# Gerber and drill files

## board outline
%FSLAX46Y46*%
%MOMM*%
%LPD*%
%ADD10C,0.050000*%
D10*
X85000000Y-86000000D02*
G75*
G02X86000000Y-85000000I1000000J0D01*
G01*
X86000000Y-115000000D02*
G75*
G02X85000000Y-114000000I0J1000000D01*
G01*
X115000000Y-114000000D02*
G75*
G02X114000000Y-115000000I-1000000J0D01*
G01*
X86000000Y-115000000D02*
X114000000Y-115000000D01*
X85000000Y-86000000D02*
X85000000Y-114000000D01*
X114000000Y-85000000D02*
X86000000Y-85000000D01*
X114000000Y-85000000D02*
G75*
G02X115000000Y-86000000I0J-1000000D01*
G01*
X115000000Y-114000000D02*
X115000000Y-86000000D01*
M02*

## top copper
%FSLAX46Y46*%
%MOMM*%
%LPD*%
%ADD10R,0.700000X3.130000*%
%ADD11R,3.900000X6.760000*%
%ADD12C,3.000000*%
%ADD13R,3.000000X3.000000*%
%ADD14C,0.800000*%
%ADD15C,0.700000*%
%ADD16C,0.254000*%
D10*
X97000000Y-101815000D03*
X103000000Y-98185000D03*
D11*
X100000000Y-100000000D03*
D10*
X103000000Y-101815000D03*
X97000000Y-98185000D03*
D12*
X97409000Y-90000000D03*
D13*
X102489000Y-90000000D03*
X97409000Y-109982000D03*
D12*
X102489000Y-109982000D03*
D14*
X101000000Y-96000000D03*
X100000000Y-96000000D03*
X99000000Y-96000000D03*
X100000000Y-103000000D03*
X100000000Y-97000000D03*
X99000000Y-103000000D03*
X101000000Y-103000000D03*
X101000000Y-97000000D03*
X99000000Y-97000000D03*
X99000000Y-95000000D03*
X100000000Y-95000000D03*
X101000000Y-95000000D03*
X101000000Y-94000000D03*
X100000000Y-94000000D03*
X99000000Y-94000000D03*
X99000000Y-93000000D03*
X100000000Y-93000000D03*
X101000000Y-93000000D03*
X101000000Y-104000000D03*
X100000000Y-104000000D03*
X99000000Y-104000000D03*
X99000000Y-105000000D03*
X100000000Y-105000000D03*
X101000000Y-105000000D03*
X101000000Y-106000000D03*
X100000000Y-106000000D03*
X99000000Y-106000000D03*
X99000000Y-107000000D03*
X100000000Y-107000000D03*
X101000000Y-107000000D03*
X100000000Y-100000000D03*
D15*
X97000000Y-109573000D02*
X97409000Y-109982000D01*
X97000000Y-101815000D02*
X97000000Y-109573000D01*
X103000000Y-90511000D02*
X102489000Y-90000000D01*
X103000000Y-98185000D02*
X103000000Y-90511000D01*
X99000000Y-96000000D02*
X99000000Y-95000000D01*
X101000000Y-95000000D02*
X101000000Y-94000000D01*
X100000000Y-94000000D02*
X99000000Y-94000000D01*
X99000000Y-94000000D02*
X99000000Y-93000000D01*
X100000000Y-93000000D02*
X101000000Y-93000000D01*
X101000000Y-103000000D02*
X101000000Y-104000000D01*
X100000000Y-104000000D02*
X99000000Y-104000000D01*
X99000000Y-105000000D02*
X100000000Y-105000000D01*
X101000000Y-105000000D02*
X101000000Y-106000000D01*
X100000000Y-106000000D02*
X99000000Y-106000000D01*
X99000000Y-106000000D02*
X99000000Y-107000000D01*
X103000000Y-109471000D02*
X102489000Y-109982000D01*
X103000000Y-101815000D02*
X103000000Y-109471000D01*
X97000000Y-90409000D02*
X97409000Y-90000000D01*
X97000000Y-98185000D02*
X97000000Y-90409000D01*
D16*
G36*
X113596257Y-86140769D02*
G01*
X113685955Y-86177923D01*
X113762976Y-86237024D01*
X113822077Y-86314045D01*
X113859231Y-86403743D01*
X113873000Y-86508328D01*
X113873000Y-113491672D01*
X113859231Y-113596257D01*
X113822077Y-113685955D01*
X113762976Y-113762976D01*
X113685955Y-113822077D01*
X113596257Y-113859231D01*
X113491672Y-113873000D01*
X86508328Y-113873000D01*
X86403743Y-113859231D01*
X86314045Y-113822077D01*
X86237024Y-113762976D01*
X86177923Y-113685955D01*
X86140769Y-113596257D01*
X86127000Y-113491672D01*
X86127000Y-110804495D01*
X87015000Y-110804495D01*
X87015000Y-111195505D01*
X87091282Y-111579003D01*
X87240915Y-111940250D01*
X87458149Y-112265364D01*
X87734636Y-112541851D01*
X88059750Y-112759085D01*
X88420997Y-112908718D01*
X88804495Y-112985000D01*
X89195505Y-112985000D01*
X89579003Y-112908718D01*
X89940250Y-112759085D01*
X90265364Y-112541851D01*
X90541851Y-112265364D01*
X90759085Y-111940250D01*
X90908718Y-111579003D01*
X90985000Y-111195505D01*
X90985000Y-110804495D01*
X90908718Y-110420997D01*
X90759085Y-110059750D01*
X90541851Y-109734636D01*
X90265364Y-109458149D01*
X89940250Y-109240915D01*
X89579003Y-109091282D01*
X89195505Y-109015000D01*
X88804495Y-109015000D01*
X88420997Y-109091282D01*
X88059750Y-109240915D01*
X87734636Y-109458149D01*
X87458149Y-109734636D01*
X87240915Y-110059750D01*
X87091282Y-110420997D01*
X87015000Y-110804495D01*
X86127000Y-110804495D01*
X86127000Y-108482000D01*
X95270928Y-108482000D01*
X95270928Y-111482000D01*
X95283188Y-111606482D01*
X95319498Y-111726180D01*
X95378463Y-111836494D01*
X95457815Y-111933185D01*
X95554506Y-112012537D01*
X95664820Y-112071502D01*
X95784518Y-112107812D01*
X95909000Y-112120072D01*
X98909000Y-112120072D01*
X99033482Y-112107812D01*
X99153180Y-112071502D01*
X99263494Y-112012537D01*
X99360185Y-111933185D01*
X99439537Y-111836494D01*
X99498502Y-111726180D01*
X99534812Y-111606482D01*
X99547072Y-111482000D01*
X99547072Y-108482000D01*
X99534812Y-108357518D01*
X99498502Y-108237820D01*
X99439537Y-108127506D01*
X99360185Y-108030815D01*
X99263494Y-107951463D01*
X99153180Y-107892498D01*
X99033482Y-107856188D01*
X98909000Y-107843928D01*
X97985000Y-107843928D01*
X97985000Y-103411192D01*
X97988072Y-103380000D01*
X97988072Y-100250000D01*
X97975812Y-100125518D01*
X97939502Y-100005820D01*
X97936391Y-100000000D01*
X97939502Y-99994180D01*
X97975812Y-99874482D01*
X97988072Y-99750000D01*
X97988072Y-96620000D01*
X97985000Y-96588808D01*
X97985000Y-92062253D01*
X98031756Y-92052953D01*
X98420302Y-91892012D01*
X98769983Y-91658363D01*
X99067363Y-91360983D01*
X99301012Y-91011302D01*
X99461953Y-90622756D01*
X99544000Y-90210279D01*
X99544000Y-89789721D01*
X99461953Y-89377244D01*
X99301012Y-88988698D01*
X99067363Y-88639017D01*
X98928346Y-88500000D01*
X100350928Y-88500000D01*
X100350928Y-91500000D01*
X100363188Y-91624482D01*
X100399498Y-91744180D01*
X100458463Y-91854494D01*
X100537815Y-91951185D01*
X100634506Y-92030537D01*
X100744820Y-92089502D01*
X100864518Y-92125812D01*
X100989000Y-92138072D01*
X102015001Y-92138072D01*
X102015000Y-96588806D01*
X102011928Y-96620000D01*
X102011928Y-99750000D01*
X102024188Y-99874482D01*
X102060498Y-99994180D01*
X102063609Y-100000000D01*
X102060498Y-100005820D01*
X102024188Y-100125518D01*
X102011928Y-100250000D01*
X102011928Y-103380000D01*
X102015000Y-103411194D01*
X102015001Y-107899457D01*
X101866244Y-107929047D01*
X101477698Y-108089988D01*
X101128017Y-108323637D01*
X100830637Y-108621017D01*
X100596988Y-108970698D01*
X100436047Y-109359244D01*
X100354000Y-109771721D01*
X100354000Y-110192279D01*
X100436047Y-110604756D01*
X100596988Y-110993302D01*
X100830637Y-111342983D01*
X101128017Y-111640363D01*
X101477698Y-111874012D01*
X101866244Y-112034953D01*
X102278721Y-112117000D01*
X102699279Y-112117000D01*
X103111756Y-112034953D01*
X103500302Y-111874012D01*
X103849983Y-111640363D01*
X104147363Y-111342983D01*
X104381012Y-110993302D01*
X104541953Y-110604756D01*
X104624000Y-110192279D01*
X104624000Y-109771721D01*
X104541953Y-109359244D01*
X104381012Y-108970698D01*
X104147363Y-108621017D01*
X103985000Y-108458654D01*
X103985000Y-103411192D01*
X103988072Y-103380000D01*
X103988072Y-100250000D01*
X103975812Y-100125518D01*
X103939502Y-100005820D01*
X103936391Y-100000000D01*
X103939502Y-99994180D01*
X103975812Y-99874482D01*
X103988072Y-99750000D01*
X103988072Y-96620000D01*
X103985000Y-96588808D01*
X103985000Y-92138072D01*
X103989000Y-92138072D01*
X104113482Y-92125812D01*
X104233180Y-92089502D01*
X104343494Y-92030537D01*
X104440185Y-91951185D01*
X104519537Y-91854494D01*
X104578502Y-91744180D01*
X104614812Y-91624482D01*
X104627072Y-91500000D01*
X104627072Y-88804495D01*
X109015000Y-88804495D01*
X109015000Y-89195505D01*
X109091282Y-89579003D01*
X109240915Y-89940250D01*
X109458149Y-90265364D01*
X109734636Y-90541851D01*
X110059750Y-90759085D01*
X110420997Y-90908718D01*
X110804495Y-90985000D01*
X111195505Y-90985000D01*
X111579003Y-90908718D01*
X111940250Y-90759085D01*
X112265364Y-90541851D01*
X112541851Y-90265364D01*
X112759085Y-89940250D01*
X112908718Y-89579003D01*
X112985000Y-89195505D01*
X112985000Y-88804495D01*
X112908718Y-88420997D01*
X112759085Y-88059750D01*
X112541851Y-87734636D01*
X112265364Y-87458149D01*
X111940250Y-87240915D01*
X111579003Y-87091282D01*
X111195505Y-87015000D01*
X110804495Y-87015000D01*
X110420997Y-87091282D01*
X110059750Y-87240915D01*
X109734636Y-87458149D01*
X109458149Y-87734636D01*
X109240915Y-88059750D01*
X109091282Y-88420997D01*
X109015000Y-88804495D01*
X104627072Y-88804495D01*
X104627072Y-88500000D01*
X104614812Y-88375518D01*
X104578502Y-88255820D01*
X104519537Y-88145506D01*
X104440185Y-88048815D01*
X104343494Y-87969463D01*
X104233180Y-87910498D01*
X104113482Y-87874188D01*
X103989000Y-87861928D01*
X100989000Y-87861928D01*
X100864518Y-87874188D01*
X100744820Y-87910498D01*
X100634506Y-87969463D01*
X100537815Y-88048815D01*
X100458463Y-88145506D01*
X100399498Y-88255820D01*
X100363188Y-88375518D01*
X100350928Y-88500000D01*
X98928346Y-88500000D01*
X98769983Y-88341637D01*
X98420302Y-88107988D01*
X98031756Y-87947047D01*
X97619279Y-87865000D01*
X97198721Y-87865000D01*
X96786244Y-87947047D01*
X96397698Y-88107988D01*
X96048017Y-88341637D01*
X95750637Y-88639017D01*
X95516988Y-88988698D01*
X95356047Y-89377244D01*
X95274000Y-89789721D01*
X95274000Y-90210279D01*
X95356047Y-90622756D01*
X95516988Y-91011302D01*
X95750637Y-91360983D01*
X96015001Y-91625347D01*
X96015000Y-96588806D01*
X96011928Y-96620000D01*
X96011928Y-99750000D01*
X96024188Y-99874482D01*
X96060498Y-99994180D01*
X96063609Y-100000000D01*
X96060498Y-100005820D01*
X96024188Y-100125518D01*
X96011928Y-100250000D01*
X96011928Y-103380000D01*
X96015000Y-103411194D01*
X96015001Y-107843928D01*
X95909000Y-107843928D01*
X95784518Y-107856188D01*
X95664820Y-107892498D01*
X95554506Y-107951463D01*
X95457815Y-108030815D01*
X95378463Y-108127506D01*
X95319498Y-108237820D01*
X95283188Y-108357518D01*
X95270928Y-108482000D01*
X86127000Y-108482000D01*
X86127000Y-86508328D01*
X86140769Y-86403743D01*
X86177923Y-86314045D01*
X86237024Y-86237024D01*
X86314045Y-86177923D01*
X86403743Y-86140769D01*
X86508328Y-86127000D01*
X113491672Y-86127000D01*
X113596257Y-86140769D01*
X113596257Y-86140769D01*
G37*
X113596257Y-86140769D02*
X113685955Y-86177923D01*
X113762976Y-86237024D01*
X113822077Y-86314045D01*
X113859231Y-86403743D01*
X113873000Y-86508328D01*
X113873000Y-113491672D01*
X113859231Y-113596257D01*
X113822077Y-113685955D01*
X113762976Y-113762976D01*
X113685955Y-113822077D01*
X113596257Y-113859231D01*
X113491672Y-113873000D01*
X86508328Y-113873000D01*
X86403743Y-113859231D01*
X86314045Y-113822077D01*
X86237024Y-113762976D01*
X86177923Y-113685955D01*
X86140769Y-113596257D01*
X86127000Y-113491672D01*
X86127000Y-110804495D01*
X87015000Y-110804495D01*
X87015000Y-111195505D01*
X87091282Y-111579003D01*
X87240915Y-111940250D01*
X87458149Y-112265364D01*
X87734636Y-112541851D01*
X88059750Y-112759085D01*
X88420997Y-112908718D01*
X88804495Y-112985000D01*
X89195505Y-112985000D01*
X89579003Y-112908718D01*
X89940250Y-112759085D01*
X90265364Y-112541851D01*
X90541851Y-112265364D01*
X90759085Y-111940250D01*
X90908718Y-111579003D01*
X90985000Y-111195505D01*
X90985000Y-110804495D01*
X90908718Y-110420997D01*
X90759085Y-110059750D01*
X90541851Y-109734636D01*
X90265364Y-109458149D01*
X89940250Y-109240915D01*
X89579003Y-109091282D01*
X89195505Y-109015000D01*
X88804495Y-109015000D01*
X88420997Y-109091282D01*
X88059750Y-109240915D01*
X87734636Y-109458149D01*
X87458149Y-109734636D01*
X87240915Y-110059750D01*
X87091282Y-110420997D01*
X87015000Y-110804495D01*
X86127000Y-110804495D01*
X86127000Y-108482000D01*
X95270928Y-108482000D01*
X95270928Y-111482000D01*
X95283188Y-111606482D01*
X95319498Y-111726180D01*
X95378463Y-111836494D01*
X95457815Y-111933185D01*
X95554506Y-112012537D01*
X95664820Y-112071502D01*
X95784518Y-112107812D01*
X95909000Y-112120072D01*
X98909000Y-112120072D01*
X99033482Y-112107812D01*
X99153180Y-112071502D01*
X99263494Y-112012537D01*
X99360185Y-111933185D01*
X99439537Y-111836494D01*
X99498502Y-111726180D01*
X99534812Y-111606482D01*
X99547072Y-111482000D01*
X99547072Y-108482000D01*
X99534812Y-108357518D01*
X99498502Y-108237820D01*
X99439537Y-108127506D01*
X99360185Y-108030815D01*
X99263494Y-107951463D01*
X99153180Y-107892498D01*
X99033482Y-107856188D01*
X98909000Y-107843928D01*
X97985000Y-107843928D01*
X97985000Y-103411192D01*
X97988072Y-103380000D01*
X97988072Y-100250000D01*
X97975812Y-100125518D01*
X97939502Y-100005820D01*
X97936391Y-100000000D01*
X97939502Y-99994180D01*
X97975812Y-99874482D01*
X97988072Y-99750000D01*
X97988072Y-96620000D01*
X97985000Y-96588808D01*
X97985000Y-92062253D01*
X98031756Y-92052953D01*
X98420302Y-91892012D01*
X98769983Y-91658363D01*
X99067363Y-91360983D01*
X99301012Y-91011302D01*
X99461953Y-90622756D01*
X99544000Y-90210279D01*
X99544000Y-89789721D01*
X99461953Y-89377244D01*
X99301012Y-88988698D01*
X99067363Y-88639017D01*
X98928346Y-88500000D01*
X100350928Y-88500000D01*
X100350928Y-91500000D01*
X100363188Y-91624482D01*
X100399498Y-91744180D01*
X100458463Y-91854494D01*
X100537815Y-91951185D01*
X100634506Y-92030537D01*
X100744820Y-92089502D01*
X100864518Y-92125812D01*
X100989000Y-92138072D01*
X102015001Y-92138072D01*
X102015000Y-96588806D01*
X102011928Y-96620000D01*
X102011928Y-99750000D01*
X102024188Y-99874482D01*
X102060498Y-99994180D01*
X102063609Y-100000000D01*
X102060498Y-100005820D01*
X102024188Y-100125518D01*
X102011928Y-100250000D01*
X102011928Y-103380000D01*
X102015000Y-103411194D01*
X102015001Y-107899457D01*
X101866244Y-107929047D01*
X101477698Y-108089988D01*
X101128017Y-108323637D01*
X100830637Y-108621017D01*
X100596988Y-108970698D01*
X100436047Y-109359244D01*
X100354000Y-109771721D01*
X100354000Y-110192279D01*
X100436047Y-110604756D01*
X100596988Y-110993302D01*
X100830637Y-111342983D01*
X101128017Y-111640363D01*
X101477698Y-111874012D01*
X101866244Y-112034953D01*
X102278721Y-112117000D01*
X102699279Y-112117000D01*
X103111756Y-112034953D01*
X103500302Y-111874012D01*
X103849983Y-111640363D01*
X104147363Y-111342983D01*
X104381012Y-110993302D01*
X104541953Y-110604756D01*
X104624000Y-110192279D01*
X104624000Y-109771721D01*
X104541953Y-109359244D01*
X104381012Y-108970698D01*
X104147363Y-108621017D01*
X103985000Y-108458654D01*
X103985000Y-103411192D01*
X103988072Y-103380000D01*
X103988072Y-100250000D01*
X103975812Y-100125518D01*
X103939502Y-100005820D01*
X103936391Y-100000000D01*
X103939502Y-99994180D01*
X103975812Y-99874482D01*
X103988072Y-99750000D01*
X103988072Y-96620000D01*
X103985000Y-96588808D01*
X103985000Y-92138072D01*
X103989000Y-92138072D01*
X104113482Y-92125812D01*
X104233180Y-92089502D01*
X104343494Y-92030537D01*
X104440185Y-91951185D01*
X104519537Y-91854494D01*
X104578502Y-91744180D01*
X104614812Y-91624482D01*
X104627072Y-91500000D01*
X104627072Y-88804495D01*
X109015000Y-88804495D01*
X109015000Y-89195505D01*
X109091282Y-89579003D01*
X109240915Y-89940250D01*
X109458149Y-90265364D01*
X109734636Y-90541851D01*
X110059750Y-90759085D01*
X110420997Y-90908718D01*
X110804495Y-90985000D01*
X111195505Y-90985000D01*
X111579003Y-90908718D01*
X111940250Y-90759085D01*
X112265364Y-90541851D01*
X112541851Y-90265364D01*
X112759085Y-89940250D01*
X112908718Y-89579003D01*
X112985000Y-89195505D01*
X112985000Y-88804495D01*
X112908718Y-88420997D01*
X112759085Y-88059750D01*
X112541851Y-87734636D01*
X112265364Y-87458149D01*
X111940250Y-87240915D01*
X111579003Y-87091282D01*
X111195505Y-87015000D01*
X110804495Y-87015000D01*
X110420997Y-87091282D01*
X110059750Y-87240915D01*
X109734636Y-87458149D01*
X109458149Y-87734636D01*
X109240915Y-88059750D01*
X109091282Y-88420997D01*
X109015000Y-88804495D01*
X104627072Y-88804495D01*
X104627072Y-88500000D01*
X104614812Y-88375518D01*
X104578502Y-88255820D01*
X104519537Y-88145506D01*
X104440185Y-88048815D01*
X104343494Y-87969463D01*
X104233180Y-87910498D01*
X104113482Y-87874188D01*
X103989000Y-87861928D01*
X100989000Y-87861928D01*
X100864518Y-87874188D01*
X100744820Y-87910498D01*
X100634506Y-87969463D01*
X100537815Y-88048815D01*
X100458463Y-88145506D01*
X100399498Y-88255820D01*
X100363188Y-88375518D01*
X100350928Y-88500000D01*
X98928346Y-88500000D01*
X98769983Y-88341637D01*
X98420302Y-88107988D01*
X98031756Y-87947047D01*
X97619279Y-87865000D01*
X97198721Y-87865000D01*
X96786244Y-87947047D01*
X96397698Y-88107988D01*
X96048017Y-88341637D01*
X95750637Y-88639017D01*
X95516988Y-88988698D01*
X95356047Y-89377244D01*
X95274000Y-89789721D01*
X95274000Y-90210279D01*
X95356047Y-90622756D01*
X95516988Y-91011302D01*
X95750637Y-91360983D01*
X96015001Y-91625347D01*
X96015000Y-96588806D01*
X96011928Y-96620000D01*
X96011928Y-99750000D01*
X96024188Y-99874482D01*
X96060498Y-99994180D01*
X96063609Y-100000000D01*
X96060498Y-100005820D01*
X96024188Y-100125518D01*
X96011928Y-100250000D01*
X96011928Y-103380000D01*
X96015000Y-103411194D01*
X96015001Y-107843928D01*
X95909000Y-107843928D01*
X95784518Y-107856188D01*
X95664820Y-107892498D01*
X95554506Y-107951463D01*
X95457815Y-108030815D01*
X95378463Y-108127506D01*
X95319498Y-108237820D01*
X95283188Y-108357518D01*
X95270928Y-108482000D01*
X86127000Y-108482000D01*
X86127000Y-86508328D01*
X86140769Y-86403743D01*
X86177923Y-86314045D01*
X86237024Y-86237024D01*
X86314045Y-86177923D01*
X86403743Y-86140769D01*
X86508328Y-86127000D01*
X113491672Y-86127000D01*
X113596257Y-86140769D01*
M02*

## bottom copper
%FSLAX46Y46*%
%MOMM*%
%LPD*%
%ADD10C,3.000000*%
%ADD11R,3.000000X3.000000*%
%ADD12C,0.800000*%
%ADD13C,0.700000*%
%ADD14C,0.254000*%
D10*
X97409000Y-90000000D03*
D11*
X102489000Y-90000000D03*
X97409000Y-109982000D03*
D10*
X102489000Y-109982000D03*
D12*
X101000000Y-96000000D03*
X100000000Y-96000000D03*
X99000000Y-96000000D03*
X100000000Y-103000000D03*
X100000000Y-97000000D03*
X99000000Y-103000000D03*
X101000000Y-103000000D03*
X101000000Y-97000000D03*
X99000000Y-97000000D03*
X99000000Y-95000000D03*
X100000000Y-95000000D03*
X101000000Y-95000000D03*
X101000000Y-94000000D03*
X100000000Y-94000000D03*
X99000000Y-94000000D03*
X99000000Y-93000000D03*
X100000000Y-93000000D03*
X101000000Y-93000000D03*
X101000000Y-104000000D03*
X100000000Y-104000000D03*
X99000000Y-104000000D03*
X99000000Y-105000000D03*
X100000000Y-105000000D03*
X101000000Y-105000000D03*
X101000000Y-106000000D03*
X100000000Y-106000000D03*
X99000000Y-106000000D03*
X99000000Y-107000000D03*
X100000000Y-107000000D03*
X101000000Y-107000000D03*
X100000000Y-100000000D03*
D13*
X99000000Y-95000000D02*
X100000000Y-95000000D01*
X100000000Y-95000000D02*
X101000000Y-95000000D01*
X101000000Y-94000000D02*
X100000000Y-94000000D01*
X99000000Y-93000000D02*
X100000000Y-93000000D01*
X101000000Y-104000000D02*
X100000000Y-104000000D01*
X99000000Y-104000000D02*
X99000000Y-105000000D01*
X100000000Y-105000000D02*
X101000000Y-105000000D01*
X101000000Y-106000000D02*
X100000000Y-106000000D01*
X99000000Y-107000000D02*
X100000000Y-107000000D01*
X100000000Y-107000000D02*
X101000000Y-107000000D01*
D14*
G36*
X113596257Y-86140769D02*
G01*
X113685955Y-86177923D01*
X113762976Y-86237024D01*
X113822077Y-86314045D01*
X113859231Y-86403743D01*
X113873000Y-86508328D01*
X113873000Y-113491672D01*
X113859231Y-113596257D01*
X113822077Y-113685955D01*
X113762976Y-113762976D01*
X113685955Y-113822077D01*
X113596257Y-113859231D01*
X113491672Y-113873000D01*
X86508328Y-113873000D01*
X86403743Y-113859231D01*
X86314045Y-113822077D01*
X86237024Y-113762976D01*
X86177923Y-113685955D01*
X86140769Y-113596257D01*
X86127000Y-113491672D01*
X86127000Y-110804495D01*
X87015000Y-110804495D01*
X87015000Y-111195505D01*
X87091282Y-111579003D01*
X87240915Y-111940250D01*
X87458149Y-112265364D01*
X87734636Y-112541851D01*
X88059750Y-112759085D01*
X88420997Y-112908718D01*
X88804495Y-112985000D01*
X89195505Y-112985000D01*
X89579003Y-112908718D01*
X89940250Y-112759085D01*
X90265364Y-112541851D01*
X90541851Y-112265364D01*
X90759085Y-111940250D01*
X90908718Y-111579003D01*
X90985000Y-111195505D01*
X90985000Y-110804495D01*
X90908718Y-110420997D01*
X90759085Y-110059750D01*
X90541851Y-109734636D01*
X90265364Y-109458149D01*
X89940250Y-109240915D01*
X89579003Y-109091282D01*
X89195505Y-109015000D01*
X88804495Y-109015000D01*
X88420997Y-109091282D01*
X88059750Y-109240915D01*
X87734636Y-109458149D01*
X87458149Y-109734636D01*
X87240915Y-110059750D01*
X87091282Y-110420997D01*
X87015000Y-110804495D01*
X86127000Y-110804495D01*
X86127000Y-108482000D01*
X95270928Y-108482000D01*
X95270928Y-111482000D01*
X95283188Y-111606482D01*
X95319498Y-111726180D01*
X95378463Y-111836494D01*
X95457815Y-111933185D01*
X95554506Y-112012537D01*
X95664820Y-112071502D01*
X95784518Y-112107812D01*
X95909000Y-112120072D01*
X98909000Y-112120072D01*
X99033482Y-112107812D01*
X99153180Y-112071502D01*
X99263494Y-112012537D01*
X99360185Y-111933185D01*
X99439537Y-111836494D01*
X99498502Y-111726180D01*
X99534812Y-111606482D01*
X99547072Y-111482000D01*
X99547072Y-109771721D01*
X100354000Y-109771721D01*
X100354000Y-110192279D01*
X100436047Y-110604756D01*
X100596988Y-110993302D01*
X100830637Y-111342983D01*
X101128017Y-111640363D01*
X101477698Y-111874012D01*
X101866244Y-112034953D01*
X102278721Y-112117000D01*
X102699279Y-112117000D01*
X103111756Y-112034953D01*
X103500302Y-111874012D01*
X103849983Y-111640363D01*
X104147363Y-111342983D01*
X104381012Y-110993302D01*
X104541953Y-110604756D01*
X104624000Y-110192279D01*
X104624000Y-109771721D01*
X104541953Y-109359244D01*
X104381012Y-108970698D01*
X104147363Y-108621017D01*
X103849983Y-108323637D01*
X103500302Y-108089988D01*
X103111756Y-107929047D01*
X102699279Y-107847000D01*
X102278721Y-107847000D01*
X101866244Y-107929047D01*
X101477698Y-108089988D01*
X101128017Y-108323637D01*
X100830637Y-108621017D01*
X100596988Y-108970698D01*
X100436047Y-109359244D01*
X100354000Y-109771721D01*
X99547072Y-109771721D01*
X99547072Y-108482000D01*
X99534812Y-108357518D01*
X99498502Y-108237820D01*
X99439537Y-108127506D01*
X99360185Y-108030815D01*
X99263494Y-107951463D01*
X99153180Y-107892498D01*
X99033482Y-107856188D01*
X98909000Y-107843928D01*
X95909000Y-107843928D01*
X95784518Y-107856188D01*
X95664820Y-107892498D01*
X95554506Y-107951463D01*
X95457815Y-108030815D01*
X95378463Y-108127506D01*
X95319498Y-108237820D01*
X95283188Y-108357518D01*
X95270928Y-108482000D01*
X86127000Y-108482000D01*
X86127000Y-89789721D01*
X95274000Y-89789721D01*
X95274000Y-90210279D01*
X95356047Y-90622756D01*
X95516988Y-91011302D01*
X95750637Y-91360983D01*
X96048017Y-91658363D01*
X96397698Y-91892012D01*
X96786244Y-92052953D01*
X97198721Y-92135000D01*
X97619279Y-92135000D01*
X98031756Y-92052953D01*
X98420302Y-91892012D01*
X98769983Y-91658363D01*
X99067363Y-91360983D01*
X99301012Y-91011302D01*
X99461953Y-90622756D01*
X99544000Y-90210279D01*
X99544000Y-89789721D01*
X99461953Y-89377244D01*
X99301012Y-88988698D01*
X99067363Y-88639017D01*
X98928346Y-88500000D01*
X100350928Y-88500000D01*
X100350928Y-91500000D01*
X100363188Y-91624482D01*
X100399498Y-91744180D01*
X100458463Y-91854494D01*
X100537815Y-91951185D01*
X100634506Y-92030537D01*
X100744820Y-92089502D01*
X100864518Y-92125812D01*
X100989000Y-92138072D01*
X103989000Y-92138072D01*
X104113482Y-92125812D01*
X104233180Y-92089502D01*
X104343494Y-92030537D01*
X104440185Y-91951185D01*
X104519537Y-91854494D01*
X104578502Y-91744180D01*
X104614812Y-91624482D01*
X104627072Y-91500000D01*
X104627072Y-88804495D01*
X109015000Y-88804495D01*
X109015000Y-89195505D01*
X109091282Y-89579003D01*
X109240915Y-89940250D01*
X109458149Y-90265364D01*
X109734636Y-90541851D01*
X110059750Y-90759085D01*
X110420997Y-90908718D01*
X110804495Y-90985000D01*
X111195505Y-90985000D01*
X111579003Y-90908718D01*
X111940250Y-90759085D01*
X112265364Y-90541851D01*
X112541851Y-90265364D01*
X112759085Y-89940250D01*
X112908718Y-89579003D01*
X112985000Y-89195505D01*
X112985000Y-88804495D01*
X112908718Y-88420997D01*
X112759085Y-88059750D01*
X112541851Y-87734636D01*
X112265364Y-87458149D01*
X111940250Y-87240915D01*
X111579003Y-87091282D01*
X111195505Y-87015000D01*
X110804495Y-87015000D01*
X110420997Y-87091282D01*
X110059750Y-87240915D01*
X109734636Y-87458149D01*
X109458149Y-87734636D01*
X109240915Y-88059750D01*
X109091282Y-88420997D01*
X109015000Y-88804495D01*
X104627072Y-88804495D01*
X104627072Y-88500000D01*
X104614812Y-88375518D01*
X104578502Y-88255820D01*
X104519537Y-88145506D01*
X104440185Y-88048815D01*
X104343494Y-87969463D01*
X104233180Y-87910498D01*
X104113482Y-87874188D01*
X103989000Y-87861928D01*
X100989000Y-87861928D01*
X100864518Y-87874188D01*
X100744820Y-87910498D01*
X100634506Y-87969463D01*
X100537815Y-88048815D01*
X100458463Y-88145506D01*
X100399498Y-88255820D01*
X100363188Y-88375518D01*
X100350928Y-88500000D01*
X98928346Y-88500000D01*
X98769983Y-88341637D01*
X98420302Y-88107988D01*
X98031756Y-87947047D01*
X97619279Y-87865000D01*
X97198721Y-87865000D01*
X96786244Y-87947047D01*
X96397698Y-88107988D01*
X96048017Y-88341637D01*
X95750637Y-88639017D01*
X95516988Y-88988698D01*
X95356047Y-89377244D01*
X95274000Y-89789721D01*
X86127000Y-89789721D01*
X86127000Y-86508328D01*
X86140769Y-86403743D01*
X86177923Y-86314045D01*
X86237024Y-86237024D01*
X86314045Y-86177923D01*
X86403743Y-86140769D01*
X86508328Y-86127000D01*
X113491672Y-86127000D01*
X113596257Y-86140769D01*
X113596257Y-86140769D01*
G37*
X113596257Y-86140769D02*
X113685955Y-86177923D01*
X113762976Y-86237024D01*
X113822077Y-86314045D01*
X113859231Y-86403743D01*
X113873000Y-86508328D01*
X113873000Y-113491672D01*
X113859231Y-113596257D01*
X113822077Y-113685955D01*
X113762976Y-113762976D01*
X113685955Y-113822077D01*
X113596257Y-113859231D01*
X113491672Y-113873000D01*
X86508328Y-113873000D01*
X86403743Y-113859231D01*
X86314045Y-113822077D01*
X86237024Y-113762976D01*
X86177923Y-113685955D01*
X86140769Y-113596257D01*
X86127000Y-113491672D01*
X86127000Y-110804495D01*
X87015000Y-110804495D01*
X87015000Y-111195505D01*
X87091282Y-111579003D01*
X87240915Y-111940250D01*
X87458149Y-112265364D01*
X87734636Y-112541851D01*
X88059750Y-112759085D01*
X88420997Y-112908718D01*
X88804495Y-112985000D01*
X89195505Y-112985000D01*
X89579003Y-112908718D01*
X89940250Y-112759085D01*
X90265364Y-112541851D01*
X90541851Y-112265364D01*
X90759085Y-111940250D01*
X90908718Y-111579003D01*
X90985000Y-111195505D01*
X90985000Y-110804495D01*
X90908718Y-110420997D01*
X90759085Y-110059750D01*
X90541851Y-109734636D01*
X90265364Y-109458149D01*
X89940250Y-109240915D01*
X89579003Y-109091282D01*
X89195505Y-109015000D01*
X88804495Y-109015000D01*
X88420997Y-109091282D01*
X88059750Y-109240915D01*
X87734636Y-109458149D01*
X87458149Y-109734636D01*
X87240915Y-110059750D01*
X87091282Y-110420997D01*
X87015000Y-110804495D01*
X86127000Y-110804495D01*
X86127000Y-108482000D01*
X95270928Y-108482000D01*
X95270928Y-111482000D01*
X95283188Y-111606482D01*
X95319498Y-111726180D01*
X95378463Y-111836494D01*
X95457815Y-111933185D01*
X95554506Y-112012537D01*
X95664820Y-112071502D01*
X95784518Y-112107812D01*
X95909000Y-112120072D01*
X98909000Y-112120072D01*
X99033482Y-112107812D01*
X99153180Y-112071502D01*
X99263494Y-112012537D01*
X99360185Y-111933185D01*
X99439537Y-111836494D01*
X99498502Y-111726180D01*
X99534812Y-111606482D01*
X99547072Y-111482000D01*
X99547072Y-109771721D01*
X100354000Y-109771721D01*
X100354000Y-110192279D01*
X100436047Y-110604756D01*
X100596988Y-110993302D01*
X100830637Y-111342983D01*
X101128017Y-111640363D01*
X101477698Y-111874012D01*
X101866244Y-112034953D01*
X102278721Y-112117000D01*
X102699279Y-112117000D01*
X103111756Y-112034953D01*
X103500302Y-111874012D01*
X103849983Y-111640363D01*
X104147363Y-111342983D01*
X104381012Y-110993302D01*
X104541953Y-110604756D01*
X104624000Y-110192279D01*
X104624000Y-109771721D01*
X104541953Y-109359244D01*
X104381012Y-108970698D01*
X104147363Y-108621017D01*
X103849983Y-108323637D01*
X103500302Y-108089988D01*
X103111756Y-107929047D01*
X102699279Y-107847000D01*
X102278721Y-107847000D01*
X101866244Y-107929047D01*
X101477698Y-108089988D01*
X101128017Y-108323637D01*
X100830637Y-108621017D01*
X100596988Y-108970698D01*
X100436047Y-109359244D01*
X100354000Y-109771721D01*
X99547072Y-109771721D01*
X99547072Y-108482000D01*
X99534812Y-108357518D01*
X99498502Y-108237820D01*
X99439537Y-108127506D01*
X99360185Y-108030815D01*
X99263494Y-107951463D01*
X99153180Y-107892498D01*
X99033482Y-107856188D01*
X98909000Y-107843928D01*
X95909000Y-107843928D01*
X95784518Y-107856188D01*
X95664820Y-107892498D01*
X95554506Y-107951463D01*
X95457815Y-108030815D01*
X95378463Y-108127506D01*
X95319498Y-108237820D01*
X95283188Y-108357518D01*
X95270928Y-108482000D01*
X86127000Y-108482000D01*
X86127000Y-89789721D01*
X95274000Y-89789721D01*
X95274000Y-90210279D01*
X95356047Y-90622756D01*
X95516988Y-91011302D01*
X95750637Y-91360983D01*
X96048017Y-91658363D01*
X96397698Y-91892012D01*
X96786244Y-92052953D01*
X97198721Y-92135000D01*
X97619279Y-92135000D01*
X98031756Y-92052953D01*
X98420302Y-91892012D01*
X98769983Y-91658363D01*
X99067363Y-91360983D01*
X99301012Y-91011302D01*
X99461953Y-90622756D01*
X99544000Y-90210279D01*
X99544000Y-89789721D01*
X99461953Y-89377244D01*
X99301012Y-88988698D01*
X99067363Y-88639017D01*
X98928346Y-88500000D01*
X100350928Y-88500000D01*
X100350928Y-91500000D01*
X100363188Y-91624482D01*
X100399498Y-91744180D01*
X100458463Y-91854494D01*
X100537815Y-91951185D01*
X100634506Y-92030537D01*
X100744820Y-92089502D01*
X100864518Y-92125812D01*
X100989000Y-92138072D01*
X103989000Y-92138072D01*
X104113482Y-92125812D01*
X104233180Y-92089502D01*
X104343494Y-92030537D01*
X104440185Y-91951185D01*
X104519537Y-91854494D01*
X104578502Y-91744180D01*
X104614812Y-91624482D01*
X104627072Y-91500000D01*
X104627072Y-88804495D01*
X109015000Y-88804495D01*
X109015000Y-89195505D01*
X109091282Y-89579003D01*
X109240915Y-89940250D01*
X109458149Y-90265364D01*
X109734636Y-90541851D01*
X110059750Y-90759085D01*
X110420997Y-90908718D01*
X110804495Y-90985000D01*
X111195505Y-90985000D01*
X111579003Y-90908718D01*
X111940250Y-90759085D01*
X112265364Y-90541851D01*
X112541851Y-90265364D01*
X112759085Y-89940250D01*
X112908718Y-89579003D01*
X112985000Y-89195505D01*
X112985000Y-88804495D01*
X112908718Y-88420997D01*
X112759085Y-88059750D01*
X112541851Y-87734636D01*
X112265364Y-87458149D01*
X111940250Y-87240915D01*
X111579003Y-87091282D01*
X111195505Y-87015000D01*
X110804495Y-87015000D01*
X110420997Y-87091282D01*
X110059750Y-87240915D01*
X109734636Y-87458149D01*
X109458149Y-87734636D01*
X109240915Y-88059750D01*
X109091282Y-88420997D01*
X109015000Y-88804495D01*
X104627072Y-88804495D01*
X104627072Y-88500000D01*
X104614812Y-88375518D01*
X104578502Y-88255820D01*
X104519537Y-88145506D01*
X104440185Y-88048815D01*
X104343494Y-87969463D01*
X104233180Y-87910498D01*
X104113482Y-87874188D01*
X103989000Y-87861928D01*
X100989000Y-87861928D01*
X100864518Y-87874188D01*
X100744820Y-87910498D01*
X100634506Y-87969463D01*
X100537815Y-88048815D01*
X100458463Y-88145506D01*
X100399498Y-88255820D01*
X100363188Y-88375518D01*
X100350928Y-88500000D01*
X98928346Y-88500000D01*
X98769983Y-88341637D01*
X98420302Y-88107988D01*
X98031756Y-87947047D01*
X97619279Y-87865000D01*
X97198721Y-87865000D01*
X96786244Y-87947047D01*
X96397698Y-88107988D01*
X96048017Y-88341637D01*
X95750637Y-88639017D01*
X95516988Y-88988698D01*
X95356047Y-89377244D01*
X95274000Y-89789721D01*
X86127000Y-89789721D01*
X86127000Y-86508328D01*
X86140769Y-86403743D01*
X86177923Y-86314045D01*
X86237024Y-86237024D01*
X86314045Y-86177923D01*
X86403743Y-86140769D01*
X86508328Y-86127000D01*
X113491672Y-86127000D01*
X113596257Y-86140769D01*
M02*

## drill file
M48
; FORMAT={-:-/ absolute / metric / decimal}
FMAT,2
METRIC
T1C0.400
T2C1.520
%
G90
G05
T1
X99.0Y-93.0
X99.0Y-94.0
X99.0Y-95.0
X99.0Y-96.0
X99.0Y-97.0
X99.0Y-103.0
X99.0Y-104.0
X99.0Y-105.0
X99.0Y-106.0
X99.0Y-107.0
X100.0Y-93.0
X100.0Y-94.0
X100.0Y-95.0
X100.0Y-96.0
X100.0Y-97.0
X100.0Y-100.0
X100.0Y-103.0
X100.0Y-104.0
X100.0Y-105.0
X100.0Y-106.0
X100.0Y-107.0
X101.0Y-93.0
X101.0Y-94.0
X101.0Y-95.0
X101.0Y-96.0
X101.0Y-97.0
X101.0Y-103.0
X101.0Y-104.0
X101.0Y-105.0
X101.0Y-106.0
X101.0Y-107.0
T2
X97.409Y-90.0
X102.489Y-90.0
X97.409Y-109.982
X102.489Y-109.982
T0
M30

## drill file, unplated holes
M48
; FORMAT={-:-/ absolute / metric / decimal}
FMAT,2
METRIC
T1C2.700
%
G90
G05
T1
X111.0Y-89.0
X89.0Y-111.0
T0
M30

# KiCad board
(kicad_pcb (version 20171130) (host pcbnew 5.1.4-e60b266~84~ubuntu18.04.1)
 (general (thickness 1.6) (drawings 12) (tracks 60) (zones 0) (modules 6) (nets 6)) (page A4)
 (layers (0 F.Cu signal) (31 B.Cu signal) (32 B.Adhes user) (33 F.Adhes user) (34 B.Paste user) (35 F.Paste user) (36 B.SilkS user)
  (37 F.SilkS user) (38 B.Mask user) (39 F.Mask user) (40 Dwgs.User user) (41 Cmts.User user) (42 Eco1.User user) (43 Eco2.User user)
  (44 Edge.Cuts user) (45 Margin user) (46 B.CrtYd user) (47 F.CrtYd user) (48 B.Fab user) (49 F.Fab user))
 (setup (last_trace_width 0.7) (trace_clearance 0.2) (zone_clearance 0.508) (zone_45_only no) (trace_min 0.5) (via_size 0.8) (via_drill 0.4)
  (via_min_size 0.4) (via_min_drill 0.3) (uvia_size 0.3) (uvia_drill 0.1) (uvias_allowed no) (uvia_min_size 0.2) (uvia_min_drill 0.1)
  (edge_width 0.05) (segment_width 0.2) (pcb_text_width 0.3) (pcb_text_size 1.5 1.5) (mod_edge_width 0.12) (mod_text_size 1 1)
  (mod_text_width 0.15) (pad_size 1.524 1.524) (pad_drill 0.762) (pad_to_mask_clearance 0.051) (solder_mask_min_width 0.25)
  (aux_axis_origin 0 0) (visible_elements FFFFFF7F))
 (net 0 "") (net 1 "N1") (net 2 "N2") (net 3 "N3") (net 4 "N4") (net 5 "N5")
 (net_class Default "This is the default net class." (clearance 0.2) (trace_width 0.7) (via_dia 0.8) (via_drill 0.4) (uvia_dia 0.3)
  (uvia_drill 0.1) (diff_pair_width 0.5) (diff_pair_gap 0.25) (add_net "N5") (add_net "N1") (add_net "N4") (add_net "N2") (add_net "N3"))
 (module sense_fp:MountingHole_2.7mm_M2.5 (layer F.Cu) (at 111 89)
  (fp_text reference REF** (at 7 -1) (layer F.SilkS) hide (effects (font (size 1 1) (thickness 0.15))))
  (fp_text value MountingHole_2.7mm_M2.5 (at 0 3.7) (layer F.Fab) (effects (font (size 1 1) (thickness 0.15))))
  (pad 1 np_thru_hole circle (at 0 0) (size 2.7 2.7) (drill 2.7) (layers *.Cu *.Mask)))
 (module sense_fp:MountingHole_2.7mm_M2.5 (layer F.Cu) (at 89 111)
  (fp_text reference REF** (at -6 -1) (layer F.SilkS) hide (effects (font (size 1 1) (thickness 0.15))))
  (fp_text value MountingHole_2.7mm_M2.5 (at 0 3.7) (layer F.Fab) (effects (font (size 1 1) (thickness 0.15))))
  (pad 1 np_thru_hole circle (at 0 0) (size 2.7 2.7) (drill 2.7) (layers *.Cu *.Mask)))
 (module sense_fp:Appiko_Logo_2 (layer F.Cu) (at 90 102 90)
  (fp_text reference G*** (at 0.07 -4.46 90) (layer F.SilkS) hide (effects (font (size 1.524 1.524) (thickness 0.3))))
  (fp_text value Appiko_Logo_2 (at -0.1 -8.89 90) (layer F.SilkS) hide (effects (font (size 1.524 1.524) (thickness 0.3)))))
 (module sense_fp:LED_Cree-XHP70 (layer F.Cu) (at 100 100)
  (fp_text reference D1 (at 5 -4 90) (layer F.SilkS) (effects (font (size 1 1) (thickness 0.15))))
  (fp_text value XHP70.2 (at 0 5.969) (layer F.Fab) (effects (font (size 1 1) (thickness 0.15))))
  (pad 2 smd rect (at -3 1.815) (size 0.7 3.13) (layers F.Cu F.Paste F.Mask) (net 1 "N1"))
  (pad 4 smd rect (at 3 -1.815) (size 0.7 3.13) (layers F.Cu F.Paste F.Mask) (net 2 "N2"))
  (pad 5 smd rect (at 0 0) (size 3.9 6.76) (layers F.Cu F.Mask) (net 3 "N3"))
  (pad 3 smd rect (at 3 1.815) (size 0.7 3.13) (layers F.Cu B.Paste F.Mask) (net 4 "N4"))
  (pad 1 smd rect (at -3 -1.815) (size 0.7 3.13) (layers F.Cu F.Paste F.Mask) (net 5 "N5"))
  (pad 3 smd rect (at -0.77 -2.31) (size 1.29 1.29) (layers F.Paste) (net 4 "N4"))
  (pad 3 smd rect (at 0.77 -2.31) (size 1.29 1.29) (layers F.Paste) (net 4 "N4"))
  (pad 3 smd rect (at -0.77 -0.77) (size 1.29 1.29) (layers F.Paste) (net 4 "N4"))
  (pad 3 smd rect (at 0.77 -0.77) (size 1.29 1.29) (layers F.Paste) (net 4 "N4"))
  (pad 3 smd rect (at -0.77 0.77) (size 1.29 1.29) (layers F.Paste) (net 4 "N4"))
  (pad 3 smd rect (at 0.77 0.77) (size 1.29 1.29) (layers F.Paste) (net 4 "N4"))
  (pad 3 smd rect (at -0.77 2.31) (size 1.29 1.29) (layers F.Paste) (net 4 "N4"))
  (pad 3 smd rect (at 0.77 2.31) (size 1.29 1.29) (layers F.Paste) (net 4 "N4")))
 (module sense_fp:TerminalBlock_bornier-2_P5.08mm (layer F.Cu) (at 102.489 90 180)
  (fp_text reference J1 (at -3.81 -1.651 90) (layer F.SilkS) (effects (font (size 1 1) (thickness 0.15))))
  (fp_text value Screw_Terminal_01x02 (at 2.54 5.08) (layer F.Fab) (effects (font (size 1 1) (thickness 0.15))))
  (pad 2 thru_hole circle (at 5.08 0 180) (size 3 3) (drill 1.52) (layers *.Cu *.Mask) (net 5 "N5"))
  (pad 1 thru_hole rect (at 0 0 180) (size 3 3) (drill 1.52) (layers *.Cu *.Mask) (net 2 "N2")))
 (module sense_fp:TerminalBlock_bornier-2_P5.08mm (layer F.Cu) (at 97.409 109.982)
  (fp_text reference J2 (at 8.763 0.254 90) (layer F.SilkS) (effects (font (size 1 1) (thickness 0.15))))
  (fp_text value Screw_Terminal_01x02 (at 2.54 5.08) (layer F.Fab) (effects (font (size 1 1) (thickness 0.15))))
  (pad 1 thru_hole rect (at 0 0) (size 3 3) (drill 1.52) (layers *.Cu *.Mask) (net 1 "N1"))
  (pad 2 thru_hole circle (at 5.08 0) (size 3 3) (drill 1.52) (layers *.Cu *.Mask) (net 4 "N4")))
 (gr_arc (start 86 86) (end 86 85) (angle -90) (layer Edge.Cuts) (width 0.05))
 (gr_arc (start 86 114) (end 85 114) (angle -90) (layer Edge.Cuts) (width 0.05))
 (gr_arc (start 114 114) (end 114 115) (angle -90) (layer Edge.Cuts) (width 0.05))
 (gr_line (start 86 115) (end 114 115) (layer Edge.Cuts) (width 0.05))
 (gr_line (start 85 86) (end 85 114) (layer Edge.Cuts) (width 0.05))
 (gr_line (start 114 85) (end 86 85) (layer Edge.Cuts) (width 0.05))
 (gr_arc (start 114 86) (end 115 86) (angle -90) (layer Edge.Cuts) (width 0.05))
 (gr_line (start 115 114) (end 115 86) (layer Edge.Cuts) (width 0.05))
 (segment (start 97 109.573) (end 97.409 109.982) (width 0.7) (layer F.Cu) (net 1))
 (segment (start 97 101.815) (end 97 109.573) (width 0.7) (layer F.Cu) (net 1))
 (segment (start 103 90.511) (end 102.489 90) (width 0.7) (layer F.Cu) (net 2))
 (segment (start 103 98.185) (end 103 90.511) (width 0.7) (layer F.Cu) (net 2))
 (via (at 101 96) (size 0.8) (drill 0.4) (layers F.Cu B.Cu) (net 3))
 (via (at 100 96) (size 0.8) (drill 0.4) (layers F.Cu B.Cu) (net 3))
 (via (at 99 96) (size 0.8) (drill 0.4) (layers F.Cu B.Cu) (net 3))
 (via (at 100 103) (size 0.8) (drill 0.4) (layers F.Cu B.Cu) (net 3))
 (via (at 100 97) (size 0.8) (drill 0.4) (layers F.Cu B.Cu) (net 3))
 (via (at 99 103) (size 0.8) (drill 0.4) (layers F.Cu B.Cu) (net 3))
 (via (at 101 103) (size 0.8) (drill 0.4) (layers F.Cu B.Cu) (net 3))
 (via (at 101 97) (size 0.8) (drill 0.4) (layers F.Cu B.Cu) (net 3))
 (via (at 99 97) (size 0.8) (drill 0.4) (layers F.Cu B.Cu) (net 3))
 (via (at 99 95) (size 0.8) (drill 0.4) (layers F.Cu B.Cu) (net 3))
 (segment (start 99 96) (end 99 95) (width 0.7) (layer F.Cu) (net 3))
 (segment (start 99 95) (end 100 95) (width 0.7) (layer B.Cu) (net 3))
 (via (at 100 95) (size 0.8) (drill 0.4) (layers F.Cu B.Cu) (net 3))
 (via (at 101 95) (size 0.8) (drill 0.4) (layers F.Cu B.Cu) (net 3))
 (segment (start 100 95) (end 101 95) (width 0.7) (layer B.Cu) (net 3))
 (via (at 101 94) (size 0.8) (drill 0.4) (layers F.Cu B.Cu) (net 3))
 (segment (start 101 95) (end 101 94) (width 0.7) (layer F.Cu) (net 3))
 (via (at 100 94) (size 0.8) (drill 0.4) (layers F.Cu B.Cu) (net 3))
 (segment (start 101 94) (end 100 94) (width 0.7) (layer B.Cu) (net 3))
 (segment (start 100 94) (end 99 94) (width 0.7) (layer F.Cu) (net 3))
 (via (at 99 94) (size 0.8) (drill 0.4) (layers F.Cu B.Cu) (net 3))
 (via (at 99 93) (size 0.8) (drill 0.4) (layers F.Cu B.Cu) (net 3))
 (segment (start 99 94) (end 99 93) (width 0.7) (layer F.Cu) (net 3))
 (via (at 100 93) (size 0.8) (drill 0.4) (layers F.Cu B.Cu) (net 3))
 (segment (start 99 93) (end 100 93) (width 0.7) (layer B.Cu) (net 3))
 (via (at 101 93) (size 0.8) (drill 0.4) (layers F.Cu B.Cu) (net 3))
 (segment (start 100 93) (end 101 93) (width 0.7) (layer F.Cu) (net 3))
 (via (at 101 104) (size 0.8) (drill 0.4) (layers F.Cu B.Cu) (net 3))
 (segment (start 101 103) (end 101 104) (width 0.7) (layer F.Cu) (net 3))
 (via (at 100 104) (size 0.8) (drill 0.4) (layers F.Cu B.Cu) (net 3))
 (segment (start 101 104) (end 100 104) (width 0.7) (layer B.Cu) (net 3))
 (via (at 99 104) (size 0.8) (drill 0.4) (layers F.Cu B.Cu) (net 3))
 (segment (start 100 104) (end 99 104) (width 0.7) (layer F.Cu) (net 3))
 (via (at 99 105) (size 0.8) (drill 0.4) (layers F.Cu B.Cu) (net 3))
 (segment (start 99 104) (end 99 105) (width 0.7) (layer B.Cu) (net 3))
 (via (at 100 105) (size 0.8) (drill 0.4) (layers F.Cu B.Cu) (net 3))
 (segment (start 99 105) (end 100 105) (width 0.7) (layer F.Cu) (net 3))
 (via (at 101 105) (size 0.8) (drill 0.4) (layers F.Cu B.Cu) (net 3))
 (segment (start 100 105) (end 101 105) (width 0.7) (layer B.Cu) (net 3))
 (via (at 101 106) (size 0.8) (drill 0.4) (layers F.Cu B.Cu) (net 3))
 (segment (start 101 105) (end 101 106) (width 0.7) (layer F.Cu) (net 3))
 (via (at 100 106) (size 0.8) (drill 0.4) (layers F.Cu B.Cu) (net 3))
 (segment (start 101 106) (end 100 106) (width 0.7) (layer B.Cu) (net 3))
 (segment (start 100 106) (end 99 106) (width 0.7) (layer F.Cu) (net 3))
 (via (at 99 106) (size 0.8) (drill 0.4) (layers F.Cu B.Cu) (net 3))
 (via (at 99 107) (size 0.8) (drill 0.4) (layers F.Cu B.Cu) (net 3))
 (segment (start 99 106) (end 99 107) (width 0.7) (layer F.Cu) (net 3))
 (segment (start 99 107) (end 100 107) (width 0.7) (layer B.Cu) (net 3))
 (via (at 100 107) (size 0.8) (drill 0.4) (layers F.Cu B.Cu) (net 3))
 (via (at 101 107) (size 0.8) (drill 0.4) (layers F.Cu B.Cu) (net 3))
 (segment (start 100 107) (end 101 107) (width 0.7) (layer B.Cu) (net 3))
 (via (at 100 100) (size 0.8) (drill 0.4) (layers F.Cu B.Cu) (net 3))
 (segment (start 103 109.471) (end 102.489 109.982) (width 0.7) (layer F.Cu) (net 4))
 (segment (start 103 101.815) (end 103 109.471) (width 0.7) (layer F.Cu) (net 4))
 (segment (start 97 90.409) (end 97.409 90) (width 0.7) (layer F.Cu) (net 5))
 (segment (start 97 98.185) (end 97 90.409) (width 0.7) (layer F.Cu) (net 5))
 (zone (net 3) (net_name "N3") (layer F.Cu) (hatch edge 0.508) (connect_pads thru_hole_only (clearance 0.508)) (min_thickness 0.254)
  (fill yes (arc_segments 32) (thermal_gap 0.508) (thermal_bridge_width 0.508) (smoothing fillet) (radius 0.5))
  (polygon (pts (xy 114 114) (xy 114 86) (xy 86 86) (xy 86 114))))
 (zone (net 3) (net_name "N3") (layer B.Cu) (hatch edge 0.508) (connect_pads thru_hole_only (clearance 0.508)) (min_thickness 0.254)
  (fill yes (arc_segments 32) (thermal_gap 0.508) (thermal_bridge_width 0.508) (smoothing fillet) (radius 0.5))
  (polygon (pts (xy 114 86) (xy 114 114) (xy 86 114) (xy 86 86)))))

